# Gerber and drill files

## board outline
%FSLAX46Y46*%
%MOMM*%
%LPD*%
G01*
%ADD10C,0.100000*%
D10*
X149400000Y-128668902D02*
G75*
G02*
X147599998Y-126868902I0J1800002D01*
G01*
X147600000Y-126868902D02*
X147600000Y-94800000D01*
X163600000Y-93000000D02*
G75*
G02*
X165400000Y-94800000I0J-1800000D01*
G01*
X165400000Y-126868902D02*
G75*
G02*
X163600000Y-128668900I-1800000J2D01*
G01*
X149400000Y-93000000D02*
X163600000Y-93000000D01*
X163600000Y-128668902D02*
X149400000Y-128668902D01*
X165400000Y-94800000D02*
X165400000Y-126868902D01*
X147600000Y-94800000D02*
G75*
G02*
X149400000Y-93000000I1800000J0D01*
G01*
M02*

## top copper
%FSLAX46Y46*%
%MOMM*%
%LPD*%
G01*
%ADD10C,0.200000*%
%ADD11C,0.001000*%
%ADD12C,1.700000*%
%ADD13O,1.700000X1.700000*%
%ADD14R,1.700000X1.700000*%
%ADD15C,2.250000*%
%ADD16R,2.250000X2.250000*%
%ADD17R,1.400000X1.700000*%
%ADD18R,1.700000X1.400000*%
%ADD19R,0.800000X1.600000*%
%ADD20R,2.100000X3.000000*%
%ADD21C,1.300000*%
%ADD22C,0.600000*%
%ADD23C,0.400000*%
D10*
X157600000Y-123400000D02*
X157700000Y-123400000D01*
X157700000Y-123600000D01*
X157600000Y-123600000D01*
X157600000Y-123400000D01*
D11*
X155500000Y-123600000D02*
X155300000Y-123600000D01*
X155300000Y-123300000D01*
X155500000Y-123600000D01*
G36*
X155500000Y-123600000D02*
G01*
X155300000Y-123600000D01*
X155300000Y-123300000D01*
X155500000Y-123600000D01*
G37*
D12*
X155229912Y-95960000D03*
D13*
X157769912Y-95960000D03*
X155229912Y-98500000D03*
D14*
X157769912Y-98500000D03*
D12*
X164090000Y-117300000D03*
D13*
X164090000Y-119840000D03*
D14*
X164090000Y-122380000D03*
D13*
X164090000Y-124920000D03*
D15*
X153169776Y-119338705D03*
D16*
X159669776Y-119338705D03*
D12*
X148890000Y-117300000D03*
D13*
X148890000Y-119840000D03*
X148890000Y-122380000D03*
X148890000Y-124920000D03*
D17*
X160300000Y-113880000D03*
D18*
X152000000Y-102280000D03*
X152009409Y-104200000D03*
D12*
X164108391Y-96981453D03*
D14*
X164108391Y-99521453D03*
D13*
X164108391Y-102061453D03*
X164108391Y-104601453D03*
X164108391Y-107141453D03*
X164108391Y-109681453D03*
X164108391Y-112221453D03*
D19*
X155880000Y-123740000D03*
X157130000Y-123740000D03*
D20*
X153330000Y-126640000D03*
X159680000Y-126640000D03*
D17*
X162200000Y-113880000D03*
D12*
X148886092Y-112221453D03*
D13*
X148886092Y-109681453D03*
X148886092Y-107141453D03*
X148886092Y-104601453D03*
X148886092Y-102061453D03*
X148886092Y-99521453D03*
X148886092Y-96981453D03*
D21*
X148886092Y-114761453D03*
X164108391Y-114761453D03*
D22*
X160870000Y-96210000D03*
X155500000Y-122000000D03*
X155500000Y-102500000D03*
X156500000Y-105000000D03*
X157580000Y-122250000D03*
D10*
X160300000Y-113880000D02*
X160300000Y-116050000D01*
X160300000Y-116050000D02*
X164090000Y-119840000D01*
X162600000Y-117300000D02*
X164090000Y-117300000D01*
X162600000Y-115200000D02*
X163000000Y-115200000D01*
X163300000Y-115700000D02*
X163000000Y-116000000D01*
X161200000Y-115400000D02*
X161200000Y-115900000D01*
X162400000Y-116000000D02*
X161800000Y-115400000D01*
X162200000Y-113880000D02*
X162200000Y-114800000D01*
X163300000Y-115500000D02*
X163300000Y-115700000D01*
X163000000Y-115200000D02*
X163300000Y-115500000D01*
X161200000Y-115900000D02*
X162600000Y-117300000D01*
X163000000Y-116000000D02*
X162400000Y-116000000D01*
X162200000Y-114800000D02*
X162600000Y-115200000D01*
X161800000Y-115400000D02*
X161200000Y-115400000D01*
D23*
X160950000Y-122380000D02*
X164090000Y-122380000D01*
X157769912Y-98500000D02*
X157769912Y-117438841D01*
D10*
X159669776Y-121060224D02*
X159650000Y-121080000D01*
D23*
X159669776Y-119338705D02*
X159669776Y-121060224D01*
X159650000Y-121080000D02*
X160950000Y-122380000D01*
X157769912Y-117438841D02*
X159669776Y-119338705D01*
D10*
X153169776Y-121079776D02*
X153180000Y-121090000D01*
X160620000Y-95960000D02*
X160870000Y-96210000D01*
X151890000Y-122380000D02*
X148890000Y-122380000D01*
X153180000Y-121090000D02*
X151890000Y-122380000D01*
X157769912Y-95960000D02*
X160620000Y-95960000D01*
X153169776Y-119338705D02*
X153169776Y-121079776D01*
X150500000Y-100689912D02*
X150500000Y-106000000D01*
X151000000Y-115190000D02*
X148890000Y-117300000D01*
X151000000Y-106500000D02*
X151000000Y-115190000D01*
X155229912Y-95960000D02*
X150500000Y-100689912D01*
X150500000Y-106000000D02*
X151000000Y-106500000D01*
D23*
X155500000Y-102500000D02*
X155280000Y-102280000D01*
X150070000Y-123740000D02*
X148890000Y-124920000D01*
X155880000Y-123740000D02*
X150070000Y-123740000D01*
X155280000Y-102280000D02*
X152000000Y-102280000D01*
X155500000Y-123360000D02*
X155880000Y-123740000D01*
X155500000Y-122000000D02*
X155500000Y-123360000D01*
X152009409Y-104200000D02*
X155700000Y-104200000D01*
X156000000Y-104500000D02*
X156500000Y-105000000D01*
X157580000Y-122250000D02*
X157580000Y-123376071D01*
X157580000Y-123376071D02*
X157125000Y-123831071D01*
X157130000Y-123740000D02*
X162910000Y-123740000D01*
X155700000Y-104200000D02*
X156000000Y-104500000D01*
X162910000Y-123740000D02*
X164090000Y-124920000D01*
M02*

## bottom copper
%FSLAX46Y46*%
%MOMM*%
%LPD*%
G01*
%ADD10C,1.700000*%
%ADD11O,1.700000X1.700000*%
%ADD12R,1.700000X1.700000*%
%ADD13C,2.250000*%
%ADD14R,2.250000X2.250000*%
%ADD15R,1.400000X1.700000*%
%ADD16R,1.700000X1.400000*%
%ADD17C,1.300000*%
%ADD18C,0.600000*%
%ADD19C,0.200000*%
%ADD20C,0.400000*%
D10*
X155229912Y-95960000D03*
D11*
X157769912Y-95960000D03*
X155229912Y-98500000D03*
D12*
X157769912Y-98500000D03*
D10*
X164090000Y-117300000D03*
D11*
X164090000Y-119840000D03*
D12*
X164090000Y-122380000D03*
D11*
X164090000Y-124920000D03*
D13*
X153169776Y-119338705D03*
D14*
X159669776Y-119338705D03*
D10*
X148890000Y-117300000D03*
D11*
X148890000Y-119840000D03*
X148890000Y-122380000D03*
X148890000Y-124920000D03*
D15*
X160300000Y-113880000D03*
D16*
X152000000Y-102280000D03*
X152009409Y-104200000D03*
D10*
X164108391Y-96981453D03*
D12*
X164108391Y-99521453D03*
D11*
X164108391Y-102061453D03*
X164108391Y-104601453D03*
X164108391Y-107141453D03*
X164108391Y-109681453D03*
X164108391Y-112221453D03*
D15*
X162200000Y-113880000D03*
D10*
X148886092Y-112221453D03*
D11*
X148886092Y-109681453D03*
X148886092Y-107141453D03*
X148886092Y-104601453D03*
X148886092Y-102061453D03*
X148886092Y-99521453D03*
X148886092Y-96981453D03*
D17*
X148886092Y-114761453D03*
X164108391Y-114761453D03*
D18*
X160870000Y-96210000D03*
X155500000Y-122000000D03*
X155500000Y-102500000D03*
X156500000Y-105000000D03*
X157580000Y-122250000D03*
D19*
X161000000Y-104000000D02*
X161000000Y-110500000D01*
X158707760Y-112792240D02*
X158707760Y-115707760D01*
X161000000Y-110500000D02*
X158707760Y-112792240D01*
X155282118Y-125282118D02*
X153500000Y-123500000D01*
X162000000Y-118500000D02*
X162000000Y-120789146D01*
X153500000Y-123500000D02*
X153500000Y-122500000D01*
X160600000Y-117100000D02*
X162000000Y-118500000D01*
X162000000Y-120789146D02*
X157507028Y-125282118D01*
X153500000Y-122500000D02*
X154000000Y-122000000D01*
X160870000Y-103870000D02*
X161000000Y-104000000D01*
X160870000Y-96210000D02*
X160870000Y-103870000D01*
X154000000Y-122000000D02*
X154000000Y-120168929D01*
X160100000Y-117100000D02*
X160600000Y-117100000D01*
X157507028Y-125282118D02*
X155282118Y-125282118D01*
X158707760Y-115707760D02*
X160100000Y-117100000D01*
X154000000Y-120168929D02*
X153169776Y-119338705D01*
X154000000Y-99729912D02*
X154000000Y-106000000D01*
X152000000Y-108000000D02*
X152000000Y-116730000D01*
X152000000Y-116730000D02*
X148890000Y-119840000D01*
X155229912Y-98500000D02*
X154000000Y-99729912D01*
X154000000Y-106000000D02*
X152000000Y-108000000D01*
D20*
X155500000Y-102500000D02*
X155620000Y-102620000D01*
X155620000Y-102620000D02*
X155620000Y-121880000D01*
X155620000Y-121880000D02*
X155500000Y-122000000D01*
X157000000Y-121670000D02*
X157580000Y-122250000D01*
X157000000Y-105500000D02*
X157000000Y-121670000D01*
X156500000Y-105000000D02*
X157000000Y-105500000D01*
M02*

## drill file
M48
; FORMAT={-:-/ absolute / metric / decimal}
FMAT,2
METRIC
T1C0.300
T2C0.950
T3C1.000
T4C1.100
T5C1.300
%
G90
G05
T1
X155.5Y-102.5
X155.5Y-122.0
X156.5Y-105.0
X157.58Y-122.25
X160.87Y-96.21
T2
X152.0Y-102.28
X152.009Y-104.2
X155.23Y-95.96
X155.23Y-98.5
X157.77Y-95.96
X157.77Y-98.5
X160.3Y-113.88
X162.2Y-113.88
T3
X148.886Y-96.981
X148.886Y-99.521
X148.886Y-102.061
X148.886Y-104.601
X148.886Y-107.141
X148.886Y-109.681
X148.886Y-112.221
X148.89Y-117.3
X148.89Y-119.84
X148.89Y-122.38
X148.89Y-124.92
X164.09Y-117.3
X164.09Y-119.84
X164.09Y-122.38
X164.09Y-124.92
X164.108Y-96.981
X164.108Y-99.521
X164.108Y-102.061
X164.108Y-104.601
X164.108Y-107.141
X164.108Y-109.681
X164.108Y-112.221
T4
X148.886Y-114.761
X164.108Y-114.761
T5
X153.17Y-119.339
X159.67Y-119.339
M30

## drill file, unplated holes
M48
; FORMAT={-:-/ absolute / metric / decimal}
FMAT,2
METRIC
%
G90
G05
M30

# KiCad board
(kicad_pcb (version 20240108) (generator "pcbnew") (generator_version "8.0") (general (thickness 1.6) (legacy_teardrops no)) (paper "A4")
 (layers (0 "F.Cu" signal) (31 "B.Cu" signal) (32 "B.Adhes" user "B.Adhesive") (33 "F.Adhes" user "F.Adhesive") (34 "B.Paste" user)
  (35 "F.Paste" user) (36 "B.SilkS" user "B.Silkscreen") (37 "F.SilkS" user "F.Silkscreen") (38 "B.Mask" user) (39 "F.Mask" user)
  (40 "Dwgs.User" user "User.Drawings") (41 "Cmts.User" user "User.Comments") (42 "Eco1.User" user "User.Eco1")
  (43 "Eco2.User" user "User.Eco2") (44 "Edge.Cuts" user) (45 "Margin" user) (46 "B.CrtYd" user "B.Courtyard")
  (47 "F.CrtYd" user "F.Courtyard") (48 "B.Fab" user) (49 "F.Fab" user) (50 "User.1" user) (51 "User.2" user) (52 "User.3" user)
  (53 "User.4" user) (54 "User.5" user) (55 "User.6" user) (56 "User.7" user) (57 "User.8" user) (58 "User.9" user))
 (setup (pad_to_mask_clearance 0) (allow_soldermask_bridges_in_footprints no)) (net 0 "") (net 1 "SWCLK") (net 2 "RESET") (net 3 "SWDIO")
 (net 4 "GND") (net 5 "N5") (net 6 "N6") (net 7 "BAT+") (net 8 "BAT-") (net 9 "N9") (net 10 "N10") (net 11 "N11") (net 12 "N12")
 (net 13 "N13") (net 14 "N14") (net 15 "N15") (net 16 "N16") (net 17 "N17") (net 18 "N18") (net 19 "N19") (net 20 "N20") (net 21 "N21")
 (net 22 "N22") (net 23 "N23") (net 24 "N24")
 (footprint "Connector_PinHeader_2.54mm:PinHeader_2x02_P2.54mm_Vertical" (layer "F.Cu") (at 155.229912 95.96)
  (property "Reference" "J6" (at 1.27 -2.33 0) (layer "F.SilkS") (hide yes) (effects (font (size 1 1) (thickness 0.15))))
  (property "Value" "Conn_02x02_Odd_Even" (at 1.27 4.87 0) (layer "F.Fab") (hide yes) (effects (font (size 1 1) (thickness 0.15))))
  (pad "1" thru_hole circle (at 0 0) (size 1.7 1.7) (drill 0.95) (layers "*.Cu" "*.Mask") (remove_unused_layers no) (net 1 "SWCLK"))
  (pad "2" thru_hole oval (at 2.54 0) (size 1.7 1.7) (drill 0.95) (layers "*.Cu" "*.Mask") (remove_unused_layers no) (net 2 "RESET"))
  (pad "3" thru_hole oval (at 0 2.54) (size 1.7 1.7) (drill 0.95) (layers "*.Cu" "*.Mask") (remove_unused_layers no) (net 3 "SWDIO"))
  (pad "4" thru_hole rect (at 2.54 2.54) (size 1.7 1.7) (drill 0.95) (layers "*.Cu" "*.Mask") (remove_unused_layers no) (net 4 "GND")))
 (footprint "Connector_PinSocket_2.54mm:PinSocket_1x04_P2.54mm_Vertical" (layer "F.Cu") (at 164.09 117.3)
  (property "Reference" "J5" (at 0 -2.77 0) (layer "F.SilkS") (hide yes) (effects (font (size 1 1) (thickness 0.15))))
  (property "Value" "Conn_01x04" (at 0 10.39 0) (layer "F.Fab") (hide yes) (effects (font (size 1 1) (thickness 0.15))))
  (pad "1" thru_hole circle (at 0 0) (size 1.7 1.7) (drill 1) (layers "*.Cu" "*.Mask") (remove_unused_layers no) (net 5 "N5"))
  (pad "2" thru_hole oval (at 0 2.54) (size 1.7 1.7) (drill 1) (layers "*.Cu" "*.Mask") (remove_unused_layers no) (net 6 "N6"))
  (pad "3" thru_hole rect (at 0 5.08) (size 1.7 1.7) (drill 1) (layers "*.Cu" "*.Mask") (remove_unused_layers no) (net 4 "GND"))
  (pad "4" thru_hole oval (at 0 7.62) (size 1.7 1.7) (drill 1) (layers "*.Cu" "*.Mask") (remove_unused_layers no) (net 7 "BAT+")))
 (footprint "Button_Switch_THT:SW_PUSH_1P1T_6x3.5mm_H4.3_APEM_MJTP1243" (layer "F.Cu") (at 153.169776 119.338705)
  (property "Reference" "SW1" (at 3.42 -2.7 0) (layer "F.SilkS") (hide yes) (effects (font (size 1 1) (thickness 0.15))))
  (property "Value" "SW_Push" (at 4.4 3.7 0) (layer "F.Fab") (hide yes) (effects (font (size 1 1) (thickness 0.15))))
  (pad "1" thru_hole circle (at 0 0 90) (size 2.25 2.25) (drill 1.3) (layers "*.Cu" "*.Mask") (remove_unused_layers no) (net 2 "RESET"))
  (pad "2" thru_hole rect (at 6.5 0 90) (size 2.25 2.25) (drill 1.3) (layers "*.Cu" "*.Mask") (remove_unused_layers no) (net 4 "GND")))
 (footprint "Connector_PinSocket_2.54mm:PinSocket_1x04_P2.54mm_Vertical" (layer "F.Cu") (at 148.89 117.3)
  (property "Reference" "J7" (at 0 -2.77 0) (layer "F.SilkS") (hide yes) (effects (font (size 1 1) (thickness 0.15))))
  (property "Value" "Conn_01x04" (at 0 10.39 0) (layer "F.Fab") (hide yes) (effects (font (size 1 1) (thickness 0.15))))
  (pad "1" thru_hole circle (at 0 0) (size 1.7 1.7) (drill 1) (layers "*.Cu" "*.Mask") (remove_unused_layers no) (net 1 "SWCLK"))
  (pad "2" thru_hole oval (at 0 2.54) (size 1.7 1.7) (drill 1) (layers "*.Cu" "*.Mask") (remove_unused_layers no) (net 3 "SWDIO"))
  (pad "3" thru_hole oval (at 0 5.08) (size 1.7 1.7) (drill 1) (layers "*.Cu" "*.Mask") (remove_unused_layers no) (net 2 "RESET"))
  (pad "4" thru_hole oval (at 0 7.62) (size 1.7 1.7) (drill 1) (layers "*.Cu" "*.Mask") (remove_unused_layers no) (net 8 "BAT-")))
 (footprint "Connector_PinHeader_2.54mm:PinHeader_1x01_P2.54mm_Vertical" (layer "F.Cu") (at 160.3 113.88)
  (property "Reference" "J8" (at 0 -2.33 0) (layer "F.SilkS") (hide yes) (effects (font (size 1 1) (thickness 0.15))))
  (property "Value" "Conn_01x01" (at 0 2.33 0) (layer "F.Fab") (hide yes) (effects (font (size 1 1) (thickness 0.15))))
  (pad "1" thru_hole rect (at 0 0) (size 1.4 1.7) (drill 0.95) (layers "*.Cu" "*.Mask") (remove_unused_layers no) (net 6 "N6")))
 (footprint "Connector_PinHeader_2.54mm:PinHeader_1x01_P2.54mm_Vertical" (layer "F.Cu") (at 152 102.28)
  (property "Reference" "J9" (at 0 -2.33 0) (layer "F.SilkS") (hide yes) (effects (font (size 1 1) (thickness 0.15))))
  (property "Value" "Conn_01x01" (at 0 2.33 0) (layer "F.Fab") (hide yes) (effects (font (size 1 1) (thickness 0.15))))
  (pad "1" thru_hole rect (at 0 0) (size 1.7 1.4) (drill 0.95) (layers "*.Cu" "*.Mask") (remove_unused_layers no) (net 8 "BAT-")))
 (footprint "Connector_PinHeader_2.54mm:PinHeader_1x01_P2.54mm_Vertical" (layer "F.Cu") (at 152.009409 104.2)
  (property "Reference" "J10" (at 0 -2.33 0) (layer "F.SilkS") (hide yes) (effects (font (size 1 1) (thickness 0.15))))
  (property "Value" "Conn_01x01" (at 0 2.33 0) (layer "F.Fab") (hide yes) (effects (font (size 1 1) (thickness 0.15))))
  (pad "1" thru_hole rect (at 0 0) (size 1.7 1.4) (drill 0.95) (layers "*.Cu" "*.Mask") (remove_unused_layers no) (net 7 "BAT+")))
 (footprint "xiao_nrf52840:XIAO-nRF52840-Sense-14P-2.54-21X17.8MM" (layer "F.Cu") (at 156.5 104.62)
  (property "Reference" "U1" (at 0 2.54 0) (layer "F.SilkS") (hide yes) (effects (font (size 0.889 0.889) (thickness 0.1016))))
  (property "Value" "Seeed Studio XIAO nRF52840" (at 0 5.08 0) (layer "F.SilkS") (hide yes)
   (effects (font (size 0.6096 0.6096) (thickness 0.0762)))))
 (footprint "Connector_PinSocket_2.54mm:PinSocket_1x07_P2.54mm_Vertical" (layer "F.Cu") (at 164.108391 96.981453)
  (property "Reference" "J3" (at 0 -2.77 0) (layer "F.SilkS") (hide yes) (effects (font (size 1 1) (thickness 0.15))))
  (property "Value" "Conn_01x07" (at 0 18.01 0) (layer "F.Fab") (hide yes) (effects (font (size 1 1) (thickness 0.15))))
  (pad "1" thru_hole circle (at 0 0) (size 1.7 1.7) (drill 1) (layers "*.Cu" "*.Mask") (remove_unused_layers no) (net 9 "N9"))
  (pad "2" thru_hole rect (at 0 2.54) (size 1.7 1.7) (drill 1) (layers "*.Cu" "*.Mask") (remove_unused_layers no) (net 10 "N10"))
  (pad "3" thru_hole oval (at 0 5.08) (size 1.7 1.7) (drill 1) (layers "*.Cu" "*.Mask") (remove_unused_layers no) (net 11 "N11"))
  (pad "4" thru_hole oval (at 0 7.62) (size 1.7 1.7) (drill 1) (layers "*.Cu" "*.Mask") (remove_unused_layers no) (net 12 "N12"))
  (pad "5" thru_hole oval (at 0 10.16) (size 1.7 1.7) (drill 1) (layers "*.Cu" "*.Mask") (remove_unused_layers no) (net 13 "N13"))
  (pad "6" thru_hole oval (at 0 12.7) (size 1.7 1.7) (drill 1) (layers "*.Cu" "*.Mask") (remove_unused_layers no) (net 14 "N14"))
  (pad "7" thru_hole oval (at 0 15.24) (size 1.7 1.7) (drill 1) (layers "*.Cu" "*.Mask") (remove_unused_layers no) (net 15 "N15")))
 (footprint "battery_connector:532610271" (layer "F.Cu") (at 156.505 126.04 180)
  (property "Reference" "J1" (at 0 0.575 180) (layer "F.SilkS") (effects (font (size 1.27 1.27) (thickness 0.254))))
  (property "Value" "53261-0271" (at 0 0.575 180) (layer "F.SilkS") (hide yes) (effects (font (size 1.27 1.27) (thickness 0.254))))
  (pad "1" smd rect (at 0.625 2.3 180) (size 0.8 1.6) (layers "F.Cu" "F.Paste" "F.Mask") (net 8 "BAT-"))
  (pad "2" smd rect (at -0.625 2.3 180) (size 0.8 1.6) (layers "F.Cu" "F.Paste" "F.Mask") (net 7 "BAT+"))
  (pad "MP1" smd rect (at 3.175 -0.6 180) (size 2.1 3) (layers "F.Cu" "F.Paste" "F.Mask") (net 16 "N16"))
  (pad "MP2" smd rect (at -3.175 -0.6 180) (size 2.1 3) (layers "F.Cu" "F.Paste" "F.Mask") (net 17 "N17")))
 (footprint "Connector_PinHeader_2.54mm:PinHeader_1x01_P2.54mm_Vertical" (layer "F.Cu") (at 162.2 113.88)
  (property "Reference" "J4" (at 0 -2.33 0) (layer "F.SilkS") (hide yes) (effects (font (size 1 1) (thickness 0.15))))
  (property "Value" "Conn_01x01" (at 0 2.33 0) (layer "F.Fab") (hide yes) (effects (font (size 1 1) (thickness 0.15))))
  (pad "1" thru_hole rect (at 0 0) (size 1.4 1.7) (drill 0.95) (layers "*.Cu" "*.Mask") (remove_unused_layers no) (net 5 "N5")))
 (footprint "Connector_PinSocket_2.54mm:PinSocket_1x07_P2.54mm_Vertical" (layer "F.Cu") (at 148.886092 112.221453 180)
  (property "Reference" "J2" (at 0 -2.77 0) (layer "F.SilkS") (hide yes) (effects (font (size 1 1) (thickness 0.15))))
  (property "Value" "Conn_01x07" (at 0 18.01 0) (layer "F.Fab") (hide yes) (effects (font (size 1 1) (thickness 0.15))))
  (pad "1" thru_hole circle (at 0 0 180) (size 1.7 1.7) (drill 1) (layers "*.Cu" "*.Mask") (remove_unused_layers no) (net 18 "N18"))
  (pad "2" thru_hole oval (at 0 2.54 180) (size 1.7 1.7) (drill 1) (layers "*.Cu" "*.Mask") (remove_unused_layers no) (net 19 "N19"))
  (pad "3" thru_hole oval (at 0 5.08 180) (size 1.7 1.7) (drill 1) (layers "*.Cu" "*.Mask") (remove_unused_layers no) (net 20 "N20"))
  (pad "4" thru_hole oval (at 0 7.62 180) (size 1.7 1.7) (drill 1) (layers "*.Cu" "*.Mask") (remove_unused_layers no) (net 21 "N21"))
  (pad "5" thru_hole oval (at 0 10.16 180) (size 1.7 1.7) (drill 1) (layers "*.Cu" "*.Mask") (remove_unused_layers no) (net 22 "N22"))
  (pad "6" thru_hole oval (at 0 12.7 180) (size 1.7 1.7) (drill 1) (layers "*.Cu" "*.Mask") (remove_unused_layers no) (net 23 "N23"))
  (pad "7" thru_hole oval (at 0 15.24 180) (size 1.7 1.7) (drill 1) (layers "*.Cu" "*.Mask") (remove_unused_layers no) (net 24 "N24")))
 (gr_rect (start 157.6 123.4) (end 157.7 123.6) (stroke (width 0.2) (type default)) (fill none) (layer "F.Cu") (net 7))
 (gr_poly (pts (xy 155.3 123.3) (xy 155.3 123.6) (xy 155.5 123.6)) (stroke (width 0.001) (type solid)) (fill solid) (layer "F.Cu") (net 8))
 (gr_arc (start 149.4 128.668902) (mid 148.127208 128.141694) (end 147.6 126.868902) (stroke (width 0.1) (type default)) (layer "Edge.Cuts"))
 (gr_line (start 147.6 126.868902) (end 147.6 94.8) (stroke (width 0.1) (type default)) (layer "Edge.Cuts"))
 (gr_arc (start 163.6 93) (mid 164.872792 93.527208) (end 165.4 94.8) (stroke (width 0.1) (type default)) (layer "Edge.Cuts"))
 (gr_arc (start 165.4 126.868902) (mid 164.872791 128.141693) (end 163.6 128.668902) (stroke (width 0.1) (type default)) (layer "Edge.Cuts"))
 (gr_line (start 149.4 93) (end 163.6 93) (stroke (width 0.1) (type default)) (layer "Edge.Cuts"))
 (gr_line (start 163.6 128.668902) (end 149.4 128.668902) (stroke (width 0.1) (type default)) (layer "Edge.Cuts"))
 (gr_line (start 165.4 94.8) (end 165.4 126.868902) (stroke (width 0.1) (type default)) (layer "Edge.Cuts"))
 (gr_arc (start 147.6 94.8) (mid 148.127208 93.527208) (end 149.4 93) (stroke (width 0.1) (type default)) (layer "Edge.Cuts"))
 (via (at 148.886092 114.761453) (size 1.3) (drill 1.1) (layers "F.Cu" "B.Cu") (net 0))
 (via (at 164.108391 114.761453) (size 1.3) (drill 1.1) (layers "F.Cu" "B.Cu") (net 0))
 (segment (start 160.3 113.88) (end 160.3 116.05) (width 0.2) (layer "F.Cu") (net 6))
 (segment (start 160.3 116.05) (end 164.09 119.84) (width 0.2) (layer "F.Cu") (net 6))
 (segment (start 162.6 117.3) (end 164.09 117.3) (width 0.2) (layer "F.Cu") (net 5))
 (segment (start 162.6 115.2) (end 163 115.2) (width 0.2) (layer "F.Cu") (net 5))
 (segment (start 163.3 115.7) (end 163 116) (width 0.2) (layer "F.Cu") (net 5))
 (segment (start 161.2 115.4) (end 161.2 115.9) (width 0.2) (layer "F.Cu") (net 5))
 (segment (start 162.4 116) (end 161.8 115.4) (width 0.2) (layer "F.Cu") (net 5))
 (segment (start 162.2 113.88) (end 162.2 114.8) (width 0.2) (layer "F.Cu") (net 5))
 (segment (start 163.3 115.5) (end 163.3 115.7) (width 0.2) (layer "F.Cu") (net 5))
 (segment (start 163 115.2) (end 163.3 115.5) (width 0.2) (layer "F.Cu") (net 5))
 (segment (start 161.2 115.9) (end 162.6 117.3) (width 0.2) (layer "F.Cu") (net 5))
 (segment (start 163 116) (end 162.4 116) (width 0.2) (layer "F.Cu") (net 5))
 (segment (start 162.2 114.8) (end 162.6 115.2) (width 0.2) (layer "F.Cu") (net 5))
 (segment (start 161.8 115.4) (end 161.2 115.4) (width 0.2) (layer "F.Cu") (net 5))
 (segment (start 160.95 122.38) (end 164.09 122.38) (width 0.4) (layer "F.Cu") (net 4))
 (segment (start 157.769912 98.5) (end 157.769912 117.438841) (width 0.4) (layer "F.Cu") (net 4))
 (segment (start 159.669776 121.060224) (end 159.65 121.08) (width 0.2) (layer "F.Cu") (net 4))
 (segment (start 159.669776 119.338705) (end 159.669776 121.060224) (width 0.4) (layer "F.Cu") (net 4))
 (segment (start 159.65 121.08) (end 160.95 122.38) (width 0.4) (layer "F.Cu") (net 4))
 (segment (start 157.769912 117.438841) (end 159.669776 119.338705) (width 0.4) (layer "F.Cu") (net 4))
 (segment (start 153.169776 121.079776) (end 153.18 121.09) (width 0.2) (layer "F.Cu") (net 2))
 (segment (start 160.62 95.96) (end 160.87 96.21) (width 0.2) (layer "F.Cu") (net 2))
 (segment (start 151.89 122.38) (end 148.89 122.38) (width 0.2) (layer "F.Cu") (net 2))
 (segment (start 153.18 121.09) (end 151.89 122.38) (width 0.2) (layer "F.Cu") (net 2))
 (segment (start 157.769912 95.96) (end 160.62 95.96) (width 0.2) (layer "F.Cu") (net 2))
 (segment (start 153.169776 119.338705) (end 153.169776 121.079776) (width 0.2) (layer "F.Cu") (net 2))
 (via (at 160.87 96.21) (size 0.6) (drill 0.3) (layers "F.Cu" "B.Cu") (free yes) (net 2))
 (segment (start 161 104) (end 161 110.5) (width 0.2) (layer "B.Cu") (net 2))
 (segment (start 158.70776 112.79224) (end 158.70776 115.70776) (width 0.2) (layer "B.Cu") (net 2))
 (segment (start 161 110.5) (end 158.70776 112.79224) (width 0.2) (layer "B.Cu") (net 2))
 (segment (start 155.282118 125.282118) (end 153.5 123.5) (width 0.2) (layer "B.Cu") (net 2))
 (segment (start 162 118.5) (end 162 120.789146) (width 0.2) (layer "B.Cu") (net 2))
 (segment (start 153.5 123.5) (end 153.5 122.5) (width 0.2) (layer "B.Cu") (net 2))
 (segment (start 160.6 117.1) (end 162 118.5) (width 0.2) (layer "B.Cu") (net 2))
 (segment (start 162 120.789146) (end 157.507028 125.282118) (width 0.2) (layer "B.Cu") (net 2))
 (segment (start 153.5 122.5) (end 154 122) (width 0.2) (layer "B.Cu") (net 2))
 (segment (start 160.87 103.87) (end 161 104) (width 0.2) (layer "B.Cu") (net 2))
 (segment (start 160.87 96.21) (end 160.87 103.87) (width 0.2) (layer "B.Cu") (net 2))
 (segment (start 154 122) (end 154 120.168929) (width 0.2) (layer "B.Cu") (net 2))
 (segment (start 160.1 117.1) (end 160.6 117.1) (width 0.2) (layer "B.Cu") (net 2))
 (segment (start 157.507028 125.282118) (end 155.282118 125.282118) (width 0.2) (layer "B.Cu") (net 2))
 (segment (start 158.70776 115.70776) (end 160.1 117.1) (width 0.2) (layer "B.Cu") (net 2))
 (segment (start 154 120.168929) (end 153.169776 119.338705) (width 0.2) (layer "B.Cu") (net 2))
 (segment (start 154 99.729912) (end 154 106) (width 0.2) (layer "B.Cu") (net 3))
 (segment (start 152 108) (end 152 116.73) (width 0.2) (layer "B.Cu") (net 3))
 (segment (start 152 116.73) (end 148.89 119.84) (width 0.2) (layer "B.Cu") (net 3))
 (segment (start 155.229912 98.5) (end 154 99.729912) (width 0.2) (layer "B.Cu") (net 3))
 (segment (start 154 106) (end 152 108) (width 0.2) (layer "B.Cu") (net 3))
 (segment (start 150.5 100.689912) (end 150.5 106) (width 0.2) (layer "F.Cu") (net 1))
 (segment (start 151 115.19) (end 148.89 117.3) (width 0.2) (layer "F.Cu") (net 1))
 (segment (start 151 106.5) (end 151 115.19) (width 0.2) (layer "F.Cu") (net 1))
 (segment (start 155.229912 95.96) (end 150.5 100.689912) (width 0.2) (layer "F.Cu") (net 1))
 (segment (start 150.5 106) (end 151 106.5) (width 0.2) (layer "F.Cu") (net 1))
 (segment (start 155.5 102.5) (end 155.28 102.28) (width 0.4) (layer "F.Cu") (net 8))
 (segment (start 150.07 123.74) (end 148.89 124.92) (width 0.4) (layer "F.Cu") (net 8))
 (segment (start 155.88 123.74) (end 150.07 123.74) (width 0.4) (layer "F.Cu") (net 8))
 (segment (start 155.28 102.28) (end 152 102.28) (width 0.4) (layer "F.Cu") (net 8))
 (segment (start 155.5 123.36) (end 155.88 123.74) (width 0.4) (layer "F.Cu") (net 8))
 (segment (start 155.5 122) (end 155.5 123.36) (width 0.4) (layer "F.Cu") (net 8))
 (via (at 155.5 122) (size 0.6) (drill 0.3) (layers "F.Cu" "B.Cu") (free yes) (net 8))
 (via (at 155.5 102.5) (size 0.6) (drill 0.3) (layers "F.Cu" "B.Cu") (free yes) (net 8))
 (segment (start 155.5 102.5) (end 155.62 102.62) (width 0.4) (layer "B.Cu") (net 8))
 (segment (start 155.62 102.62) (end 155.62 121.88) (width 0.4) (layer "B.Cu") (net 8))
 (segment (start 155.62 121.88) (end 155.5 122) (width 0.4) (layer "B.Cu") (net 8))
 (segment (start 152.009409 104.2) (end 155.7 104.2) (width 0.4) (layer "F.Cu") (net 7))
 (segment (start 156 104.5) (end 156.5 105) (width 0.4) (layer "F.Cu") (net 7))
 (segment (start 157.58 122.25) (end 157.58 123.376071) (width 0.4) (layer "F.Cu") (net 7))
 (segment (start 157.58 123.376071) (end 157.125 123.831071) (width 0.4) (layer "F.Cu") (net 7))
 (segment (start 157.13 123.74) (end 162.91 123.74) (width 0.4) (layer "F.Cu") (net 7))
 (segment (start 155.7 104.2) (end 156 104.5) (width 0.4) (layer "F.Cu") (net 7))
 (segment (start 162.91 123.74) (end 164.09 124.92) (width 0.4) (layer "F.Cu") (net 7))
 (via (at 156.5 105) (size 0.6) (drill 0.3) (layers "F.Cu" "B.Cu") (free yes) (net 7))
 (via (at 157.58 122.25) (size 0.6) (drill 0.3) (layers "F.Cu" "B.Cu") (free yes) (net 7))
 (segment (start 157 121.67) (end 157.58 122.25) (width 0.4) (layer "B.Cu") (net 7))
 (segment (start 157 105.5) (end 157 121.67) (width 0.4) (layer "B.Cu") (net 7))
 (segment (start 156.5 105) (end 157 105.5) (width 0.4) (layer "B.Cu") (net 7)))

